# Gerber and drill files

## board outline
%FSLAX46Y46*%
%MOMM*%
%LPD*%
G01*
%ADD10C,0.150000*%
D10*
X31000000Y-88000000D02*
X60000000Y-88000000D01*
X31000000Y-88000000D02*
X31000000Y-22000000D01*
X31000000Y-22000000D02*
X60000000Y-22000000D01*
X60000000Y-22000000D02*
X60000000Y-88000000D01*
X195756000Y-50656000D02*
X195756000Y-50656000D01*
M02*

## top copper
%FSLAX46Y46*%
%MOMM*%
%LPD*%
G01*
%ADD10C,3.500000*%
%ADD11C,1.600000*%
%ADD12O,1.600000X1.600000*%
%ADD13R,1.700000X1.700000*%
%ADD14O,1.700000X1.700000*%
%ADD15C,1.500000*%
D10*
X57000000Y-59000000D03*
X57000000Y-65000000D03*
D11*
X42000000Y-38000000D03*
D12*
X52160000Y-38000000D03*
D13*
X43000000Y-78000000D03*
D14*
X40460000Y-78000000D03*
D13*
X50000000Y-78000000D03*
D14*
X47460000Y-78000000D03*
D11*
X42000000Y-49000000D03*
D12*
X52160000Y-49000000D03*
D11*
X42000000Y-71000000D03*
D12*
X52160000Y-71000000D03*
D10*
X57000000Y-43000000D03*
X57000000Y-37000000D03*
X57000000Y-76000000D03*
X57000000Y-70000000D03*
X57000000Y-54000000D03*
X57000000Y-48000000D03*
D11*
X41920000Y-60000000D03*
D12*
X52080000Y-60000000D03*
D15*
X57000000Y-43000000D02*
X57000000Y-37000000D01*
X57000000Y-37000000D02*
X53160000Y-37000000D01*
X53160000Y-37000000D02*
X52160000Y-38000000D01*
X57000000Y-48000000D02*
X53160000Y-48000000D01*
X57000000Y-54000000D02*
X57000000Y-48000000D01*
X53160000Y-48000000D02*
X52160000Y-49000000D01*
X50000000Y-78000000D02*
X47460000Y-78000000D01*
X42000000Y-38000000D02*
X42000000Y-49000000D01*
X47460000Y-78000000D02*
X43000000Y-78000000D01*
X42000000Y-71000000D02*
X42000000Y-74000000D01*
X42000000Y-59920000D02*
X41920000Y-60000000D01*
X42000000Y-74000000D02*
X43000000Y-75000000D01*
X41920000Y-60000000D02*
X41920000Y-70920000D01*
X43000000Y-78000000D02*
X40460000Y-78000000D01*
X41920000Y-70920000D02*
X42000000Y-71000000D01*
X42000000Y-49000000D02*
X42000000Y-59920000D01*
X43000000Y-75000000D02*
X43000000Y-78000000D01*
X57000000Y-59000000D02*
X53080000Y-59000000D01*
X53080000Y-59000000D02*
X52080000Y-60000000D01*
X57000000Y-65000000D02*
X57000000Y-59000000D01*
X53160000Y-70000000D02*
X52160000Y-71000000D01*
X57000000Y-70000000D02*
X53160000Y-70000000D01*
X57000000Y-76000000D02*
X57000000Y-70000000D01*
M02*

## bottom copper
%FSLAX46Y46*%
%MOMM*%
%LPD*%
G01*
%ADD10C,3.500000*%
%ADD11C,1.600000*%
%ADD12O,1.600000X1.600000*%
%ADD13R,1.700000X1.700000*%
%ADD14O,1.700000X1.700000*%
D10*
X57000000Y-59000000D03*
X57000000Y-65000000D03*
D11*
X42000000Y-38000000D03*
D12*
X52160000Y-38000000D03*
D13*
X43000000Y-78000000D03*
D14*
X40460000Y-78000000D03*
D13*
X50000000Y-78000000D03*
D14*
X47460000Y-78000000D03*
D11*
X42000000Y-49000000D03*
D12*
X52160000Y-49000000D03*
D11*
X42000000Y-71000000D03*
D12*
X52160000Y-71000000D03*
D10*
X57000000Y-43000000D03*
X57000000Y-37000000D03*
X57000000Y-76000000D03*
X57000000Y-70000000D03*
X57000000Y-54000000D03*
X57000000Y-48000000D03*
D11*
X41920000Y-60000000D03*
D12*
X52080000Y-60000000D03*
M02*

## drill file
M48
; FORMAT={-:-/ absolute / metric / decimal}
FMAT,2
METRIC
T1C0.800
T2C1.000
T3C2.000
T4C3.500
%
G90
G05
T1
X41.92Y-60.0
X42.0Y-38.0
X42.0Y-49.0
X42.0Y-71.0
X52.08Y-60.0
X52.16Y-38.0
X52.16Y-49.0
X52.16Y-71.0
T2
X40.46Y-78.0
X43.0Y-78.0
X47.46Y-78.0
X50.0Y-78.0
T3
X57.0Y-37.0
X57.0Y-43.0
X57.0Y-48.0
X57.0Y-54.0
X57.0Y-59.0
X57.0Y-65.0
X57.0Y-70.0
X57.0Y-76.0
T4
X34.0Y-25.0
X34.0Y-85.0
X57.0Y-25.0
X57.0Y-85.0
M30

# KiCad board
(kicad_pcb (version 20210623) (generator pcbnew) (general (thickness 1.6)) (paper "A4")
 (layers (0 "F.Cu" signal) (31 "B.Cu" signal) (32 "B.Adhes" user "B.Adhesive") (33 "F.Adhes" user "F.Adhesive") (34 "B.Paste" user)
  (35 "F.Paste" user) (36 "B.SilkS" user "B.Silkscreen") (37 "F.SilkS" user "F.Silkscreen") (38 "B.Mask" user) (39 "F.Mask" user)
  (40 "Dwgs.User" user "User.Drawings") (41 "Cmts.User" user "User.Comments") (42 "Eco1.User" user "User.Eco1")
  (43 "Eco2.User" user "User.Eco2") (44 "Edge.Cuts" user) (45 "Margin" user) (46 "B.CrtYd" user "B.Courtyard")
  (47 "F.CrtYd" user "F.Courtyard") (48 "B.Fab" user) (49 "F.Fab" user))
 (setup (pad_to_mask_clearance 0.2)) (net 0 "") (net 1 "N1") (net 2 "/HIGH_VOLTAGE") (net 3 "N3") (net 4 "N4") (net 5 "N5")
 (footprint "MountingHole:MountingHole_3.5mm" (layer "F.Cu") (at 34 25)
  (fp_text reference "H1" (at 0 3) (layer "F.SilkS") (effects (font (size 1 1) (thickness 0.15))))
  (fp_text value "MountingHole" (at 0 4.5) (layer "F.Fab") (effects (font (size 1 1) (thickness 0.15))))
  (pad "1" np_thru_hole circle locked (at 0 0) (size 3.5 3.5) (drill 3.5) (layers *.Cu *.Mask)))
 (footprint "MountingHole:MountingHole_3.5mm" (layer "F.Cu") (at 57 25)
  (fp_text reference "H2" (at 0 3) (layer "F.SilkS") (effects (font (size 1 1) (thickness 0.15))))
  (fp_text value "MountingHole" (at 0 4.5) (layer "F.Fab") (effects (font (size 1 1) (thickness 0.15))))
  (pad "1" np_thru_hole circle locked (at 0 0) (size 3.5 3.5) (drill 3.5) (layers *.Cu *.Mask)))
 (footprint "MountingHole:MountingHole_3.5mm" (layer "F.Cu") (at 57 85)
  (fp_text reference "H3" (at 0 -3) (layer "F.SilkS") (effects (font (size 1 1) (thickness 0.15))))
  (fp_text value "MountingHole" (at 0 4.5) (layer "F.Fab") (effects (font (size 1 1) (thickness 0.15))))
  (pad "1" np_thru_hole circle locked (at 0 0) (size 3.5 3.5) (drill 3.5) (layers *.Cu *.Mask)))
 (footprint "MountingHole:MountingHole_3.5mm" (layer "F.Cu") (at 34 85)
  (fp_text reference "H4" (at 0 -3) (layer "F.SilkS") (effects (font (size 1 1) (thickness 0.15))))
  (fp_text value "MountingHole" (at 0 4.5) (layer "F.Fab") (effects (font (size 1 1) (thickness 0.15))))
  (pad "1" np_thru_hole circle locked (at 0 0) (size 3.5 3.5) (drill 3.5) (layers *.Cu *.Mask)))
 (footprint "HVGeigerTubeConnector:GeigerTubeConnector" (layer "F.Cu") (at 49 62 90)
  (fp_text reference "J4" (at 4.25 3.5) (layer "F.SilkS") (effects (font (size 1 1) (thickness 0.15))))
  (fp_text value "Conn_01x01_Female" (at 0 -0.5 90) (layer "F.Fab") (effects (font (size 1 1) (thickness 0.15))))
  (pad "1" thru_hole circle (at 3 8 90) (size 3.5 3.5) (drill 2) (layers *.Cu *.Mask) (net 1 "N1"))
  (pad "1" thru_hole circle (at -3 8 90) (size 3.5 3.5) (drill 2) (layers *.Cu *.Mask) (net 1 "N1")))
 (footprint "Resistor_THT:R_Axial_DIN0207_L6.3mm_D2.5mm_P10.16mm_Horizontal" (layer "F.Cu") (at 42 38)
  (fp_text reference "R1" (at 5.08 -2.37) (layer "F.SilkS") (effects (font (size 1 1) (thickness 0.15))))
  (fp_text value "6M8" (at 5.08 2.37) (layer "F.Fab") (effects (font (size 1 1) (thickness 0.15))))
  (pad "1" thru_hole circle locked (at 0 0) (size 1.6 1.6) (drill 0.8) (layers *.Cu *.Mask) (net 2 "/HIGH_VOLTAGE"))
  (pad "2" thru_hole oval locked (at 10.16 0) (size 1.6 1.6) (drill 0.8) (layers *.Cu *.Mask) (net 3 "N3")))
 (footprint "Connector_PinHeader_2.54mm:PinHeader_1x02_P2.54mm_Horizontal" (layer "F.Cu") (at 43 78 -90)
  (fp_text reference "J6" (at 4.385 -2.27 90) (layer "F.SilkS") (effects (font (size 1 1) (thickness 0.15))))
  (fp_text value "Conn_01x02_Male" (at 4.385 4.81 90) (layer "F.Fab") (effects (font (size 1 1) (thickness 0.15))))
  (pad "1" thru_hole rect locked (at 0 0 270) (size 1.7 1.7) (drill 1) (layers *.Cu *.Mask) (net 2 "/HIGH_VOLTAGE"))
  (pad "2" thru_hole oval locked (at 0 2.54 270) (size 1.7 1.7) (drill 1) (layers *.Cu *.Mask) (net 2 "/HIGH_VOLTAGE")))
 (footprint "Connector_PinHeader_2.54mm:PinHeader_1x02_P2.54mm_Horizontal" (layer "F.Cu") (at 50 78 -90)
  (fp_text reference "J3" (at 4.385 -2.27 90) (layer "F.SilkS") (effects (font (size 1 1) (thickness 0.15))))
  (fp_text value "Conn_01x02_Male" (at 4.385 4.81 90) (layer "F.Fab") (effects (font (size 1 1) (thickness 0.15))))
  (pad "1" thru_hole rect locked (at 0 0 270) (size 1.7 1.7) (drill 1) (layers *.Cu *.Mask) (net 2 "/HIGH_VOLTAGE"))
  (pad "2" thru_hole oval locked (at 0 2.54 270) (size 1.7 1.7) (drill 1) (layers *.Cu *.Mask) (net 2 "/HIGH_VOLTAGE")))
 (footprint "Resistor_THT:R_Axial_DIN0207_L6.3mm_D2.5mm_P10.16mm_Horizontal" (layer "F.Cu") (at 42 49)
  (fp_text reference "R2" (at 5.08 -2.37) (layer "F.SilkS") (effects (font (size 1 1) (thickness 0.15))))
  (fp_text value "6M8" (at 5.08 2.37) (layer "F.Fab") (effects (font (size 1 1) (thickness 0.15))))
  (pad "1" thru_hole circle locked (at 0 0) (size 1.6 1.6) (drill 0.8) (layers *.Cu *.Mask) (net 2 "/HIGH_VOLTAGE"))
  (pad "2" thru_hole oval locked (at 10.16 0) (size 1.6 1.6) (drill 0.8) (layers *.Cu *.Mask) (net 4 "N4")))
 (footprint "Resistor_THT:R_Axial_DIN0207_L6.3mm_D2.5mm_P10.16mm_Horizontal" (layer "F.Cu") (at 42 71)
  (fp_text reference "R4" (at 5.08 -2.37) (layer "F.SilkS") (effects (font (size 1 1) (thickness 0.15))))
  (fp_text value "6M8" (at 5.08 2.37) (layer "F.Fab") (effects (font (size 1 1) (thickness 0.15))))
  (pad "1" thru_hole circle locked (at 0 0) (size 1.6 1.6) (drill 0.8) (layers *.Cu *.Mask) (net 2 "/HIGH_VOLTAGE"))
  (pad "2" thru_hole oval locked (at 10.16 0) (size 1.6 1.6) (drill 0.8) (layers *.Cu *.Mask) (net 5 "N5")))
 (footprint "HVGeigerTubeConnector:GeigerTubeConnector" (layer "F.Cu") (at 49 40 90)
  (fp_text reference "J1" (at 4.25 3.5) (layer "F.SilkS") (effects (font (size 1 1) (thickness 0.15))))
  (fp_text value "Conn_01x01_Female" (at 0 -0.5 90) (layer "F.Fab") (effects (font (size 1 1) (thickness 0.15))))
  (pad "1" thru_hole circle (at -3 8 90) (size 3.5 3.5) (drill 2) (layers *.Cu *.Mask) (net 3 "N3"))
  (pad "1" thru_hole circle (at 3 8 90) (size 3.5 3.5) (drill 2) (layers *.Cu *.Mask) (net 3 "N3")))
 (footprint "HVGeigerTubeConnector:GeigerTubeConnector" (layer "F.Cu") (at 49 73 90)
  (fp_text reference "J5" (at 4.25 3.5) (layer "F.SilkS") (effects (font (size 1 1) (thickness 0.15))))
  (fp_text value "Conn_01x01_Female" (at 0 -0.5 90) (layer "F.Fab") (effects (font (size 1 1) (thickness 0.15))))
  (pad "1" thru_hole circle (at -3 8 90) (size 3.5 3.5) (drill 2) (layers *.Cu *.Mask) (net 5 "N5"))
  (pad "1" thru_hole circle (at 3 8 90) (size 3.5 3.5) (drill 2) (layers *.Cu *.Mask) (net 5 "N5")))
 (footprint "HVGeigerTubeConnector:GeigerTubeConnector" (layer "F.Cu") (at 49 51 90)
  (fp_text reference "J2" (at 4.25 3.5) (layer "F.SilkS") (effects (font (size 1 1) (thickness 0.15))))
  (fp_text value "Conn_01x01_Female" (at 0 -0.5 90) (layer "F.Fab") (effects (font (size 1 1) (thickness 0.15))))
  (pad "1" thru_hole circle (at -3 8 90) (size 3.5 3.5) (drill 2) (layers *.Cu *.Mask) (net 4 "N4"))
  (pad "1" thru_hole circle (at 3 8 90) (size 3.5 3.5) (drill 2) (layers *.Cu *.Mask) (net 4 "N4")))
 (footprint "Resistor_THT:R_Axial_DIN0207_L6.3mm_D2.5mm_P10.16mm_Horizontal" (layer "F.Cu") (at 41.92 60)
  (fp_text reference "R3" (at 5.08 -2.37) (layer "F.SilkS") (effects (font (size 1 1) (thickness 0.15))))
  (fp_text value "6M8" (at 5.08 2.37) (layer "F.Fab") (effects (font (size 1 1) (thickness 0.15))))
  (pad "1" thru_hole circle locked (at 0 0) (size 1.6 1.6) (drill 0.8) (layers *.Cu *.Mask) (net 2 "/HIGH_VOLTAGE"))
  (pad "2" thru_hole oval locked (at 10.16 0) (size 1.6 1.6) (drill 0.8) (layers *.Cu *.Mask) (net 1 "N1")))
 (gr_line (start 31 88) (end 60 88) (layer "Edge.Cuts") (width 0.15))
 (gr_line (start 31 88) (end 31 22) (layer "Edge.Cuts") (width 0.15))
 (gr_line (start 31 22) (end 60 22) (layer "Edge.Cuts") (width 0.15))
 (gr_line (start 60 22) (end 60 88) (layer "Edge.Cuts") (width 0.15))
 (gr_line (start 195.756 50.656) (end 195.756 50.656) (layer "Edge.Cuts") (width 0.15))
 (segment (start 57 43) (end 57 37) (width 1.5) (layer "F.Cu") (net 3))
 (segment (start 57 37) (end 53.16 37) (width 1.5) (layer "F.Cu") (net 3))
 (segment (start 53.16 37) (end 52.16 38) (width 1.5) (layer "F.Cu") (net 3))
 (segment (start 57 48) (end 53.16 48) (width 1.5) (layer "F.Cu") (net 4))
 (segment (start 57 54) (end 57 48) (width 1.5) (layer "F.Cu") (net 4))
 (segment (start 53.16 48) (end 52.16 49) (width 1.5) (layer "F.Cu") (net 4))
 (segment (start 50 78) (end 47.46 78) (width 1.5) (layer "F.Cu") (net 2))
 (segment (start 42 38) (end 42 49) (width 1.5) (layer "F.Cu") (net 2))
 (segment (start 47.46 78) (end 43 78) (width 1.5) (layer "F.Cu") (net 2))
 (segment (start 42 71) (end 42 74) (width 1.5) (layer "F.Cu") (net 2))
 (segment (start 42 59.92) (end 41.92 60) (width 1.5) (layer "F.Cu") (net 2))
 (segment (start 42 74) (end 43 75) (width 1.5) (layer "F.Cu") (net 2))
 (segment (start 41.92 60) (end 41.92 70.92) (width 1.5) (layer "F.Cu") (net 2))
 (segment (start 43 78) (end 40.46 78) (width 1.5) (layer "F.Cu") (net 2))
 (segment (start 41.92 70.92) (end 42 71) (width 1.5) (layer "F.Cu") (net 2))
 (segment (start 42 49) (end 42 59.92) (width 1.5) (layer "F.Cu") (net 2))
 (segment (start 43 75) (end 43 78) (width 1.5) (layer "F.Cu") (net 2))
 (segment (start 57 59) (end 53.08 59) (width 1.5) (layer "F.Cu") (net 1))
 (segment (start 53.08 59) (end 52.08 60) (width 1.5) (layer "F.Cu") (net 1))
 (segment (start 57 65) (end 57 59) (width 1.5) (layer "F.Cu") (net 1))
 (segment (start 53.16 70) (end 52.16 71) (width 1.5) (layer "F.Cu") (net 5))
 (segment (start 57 70) (end 53.16 70) (width 1.5) (layer "F.Cu") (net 5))
 (segment (start 57 76) (end 57 70) (width 1.5) (layer "F.Cu") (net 5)))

